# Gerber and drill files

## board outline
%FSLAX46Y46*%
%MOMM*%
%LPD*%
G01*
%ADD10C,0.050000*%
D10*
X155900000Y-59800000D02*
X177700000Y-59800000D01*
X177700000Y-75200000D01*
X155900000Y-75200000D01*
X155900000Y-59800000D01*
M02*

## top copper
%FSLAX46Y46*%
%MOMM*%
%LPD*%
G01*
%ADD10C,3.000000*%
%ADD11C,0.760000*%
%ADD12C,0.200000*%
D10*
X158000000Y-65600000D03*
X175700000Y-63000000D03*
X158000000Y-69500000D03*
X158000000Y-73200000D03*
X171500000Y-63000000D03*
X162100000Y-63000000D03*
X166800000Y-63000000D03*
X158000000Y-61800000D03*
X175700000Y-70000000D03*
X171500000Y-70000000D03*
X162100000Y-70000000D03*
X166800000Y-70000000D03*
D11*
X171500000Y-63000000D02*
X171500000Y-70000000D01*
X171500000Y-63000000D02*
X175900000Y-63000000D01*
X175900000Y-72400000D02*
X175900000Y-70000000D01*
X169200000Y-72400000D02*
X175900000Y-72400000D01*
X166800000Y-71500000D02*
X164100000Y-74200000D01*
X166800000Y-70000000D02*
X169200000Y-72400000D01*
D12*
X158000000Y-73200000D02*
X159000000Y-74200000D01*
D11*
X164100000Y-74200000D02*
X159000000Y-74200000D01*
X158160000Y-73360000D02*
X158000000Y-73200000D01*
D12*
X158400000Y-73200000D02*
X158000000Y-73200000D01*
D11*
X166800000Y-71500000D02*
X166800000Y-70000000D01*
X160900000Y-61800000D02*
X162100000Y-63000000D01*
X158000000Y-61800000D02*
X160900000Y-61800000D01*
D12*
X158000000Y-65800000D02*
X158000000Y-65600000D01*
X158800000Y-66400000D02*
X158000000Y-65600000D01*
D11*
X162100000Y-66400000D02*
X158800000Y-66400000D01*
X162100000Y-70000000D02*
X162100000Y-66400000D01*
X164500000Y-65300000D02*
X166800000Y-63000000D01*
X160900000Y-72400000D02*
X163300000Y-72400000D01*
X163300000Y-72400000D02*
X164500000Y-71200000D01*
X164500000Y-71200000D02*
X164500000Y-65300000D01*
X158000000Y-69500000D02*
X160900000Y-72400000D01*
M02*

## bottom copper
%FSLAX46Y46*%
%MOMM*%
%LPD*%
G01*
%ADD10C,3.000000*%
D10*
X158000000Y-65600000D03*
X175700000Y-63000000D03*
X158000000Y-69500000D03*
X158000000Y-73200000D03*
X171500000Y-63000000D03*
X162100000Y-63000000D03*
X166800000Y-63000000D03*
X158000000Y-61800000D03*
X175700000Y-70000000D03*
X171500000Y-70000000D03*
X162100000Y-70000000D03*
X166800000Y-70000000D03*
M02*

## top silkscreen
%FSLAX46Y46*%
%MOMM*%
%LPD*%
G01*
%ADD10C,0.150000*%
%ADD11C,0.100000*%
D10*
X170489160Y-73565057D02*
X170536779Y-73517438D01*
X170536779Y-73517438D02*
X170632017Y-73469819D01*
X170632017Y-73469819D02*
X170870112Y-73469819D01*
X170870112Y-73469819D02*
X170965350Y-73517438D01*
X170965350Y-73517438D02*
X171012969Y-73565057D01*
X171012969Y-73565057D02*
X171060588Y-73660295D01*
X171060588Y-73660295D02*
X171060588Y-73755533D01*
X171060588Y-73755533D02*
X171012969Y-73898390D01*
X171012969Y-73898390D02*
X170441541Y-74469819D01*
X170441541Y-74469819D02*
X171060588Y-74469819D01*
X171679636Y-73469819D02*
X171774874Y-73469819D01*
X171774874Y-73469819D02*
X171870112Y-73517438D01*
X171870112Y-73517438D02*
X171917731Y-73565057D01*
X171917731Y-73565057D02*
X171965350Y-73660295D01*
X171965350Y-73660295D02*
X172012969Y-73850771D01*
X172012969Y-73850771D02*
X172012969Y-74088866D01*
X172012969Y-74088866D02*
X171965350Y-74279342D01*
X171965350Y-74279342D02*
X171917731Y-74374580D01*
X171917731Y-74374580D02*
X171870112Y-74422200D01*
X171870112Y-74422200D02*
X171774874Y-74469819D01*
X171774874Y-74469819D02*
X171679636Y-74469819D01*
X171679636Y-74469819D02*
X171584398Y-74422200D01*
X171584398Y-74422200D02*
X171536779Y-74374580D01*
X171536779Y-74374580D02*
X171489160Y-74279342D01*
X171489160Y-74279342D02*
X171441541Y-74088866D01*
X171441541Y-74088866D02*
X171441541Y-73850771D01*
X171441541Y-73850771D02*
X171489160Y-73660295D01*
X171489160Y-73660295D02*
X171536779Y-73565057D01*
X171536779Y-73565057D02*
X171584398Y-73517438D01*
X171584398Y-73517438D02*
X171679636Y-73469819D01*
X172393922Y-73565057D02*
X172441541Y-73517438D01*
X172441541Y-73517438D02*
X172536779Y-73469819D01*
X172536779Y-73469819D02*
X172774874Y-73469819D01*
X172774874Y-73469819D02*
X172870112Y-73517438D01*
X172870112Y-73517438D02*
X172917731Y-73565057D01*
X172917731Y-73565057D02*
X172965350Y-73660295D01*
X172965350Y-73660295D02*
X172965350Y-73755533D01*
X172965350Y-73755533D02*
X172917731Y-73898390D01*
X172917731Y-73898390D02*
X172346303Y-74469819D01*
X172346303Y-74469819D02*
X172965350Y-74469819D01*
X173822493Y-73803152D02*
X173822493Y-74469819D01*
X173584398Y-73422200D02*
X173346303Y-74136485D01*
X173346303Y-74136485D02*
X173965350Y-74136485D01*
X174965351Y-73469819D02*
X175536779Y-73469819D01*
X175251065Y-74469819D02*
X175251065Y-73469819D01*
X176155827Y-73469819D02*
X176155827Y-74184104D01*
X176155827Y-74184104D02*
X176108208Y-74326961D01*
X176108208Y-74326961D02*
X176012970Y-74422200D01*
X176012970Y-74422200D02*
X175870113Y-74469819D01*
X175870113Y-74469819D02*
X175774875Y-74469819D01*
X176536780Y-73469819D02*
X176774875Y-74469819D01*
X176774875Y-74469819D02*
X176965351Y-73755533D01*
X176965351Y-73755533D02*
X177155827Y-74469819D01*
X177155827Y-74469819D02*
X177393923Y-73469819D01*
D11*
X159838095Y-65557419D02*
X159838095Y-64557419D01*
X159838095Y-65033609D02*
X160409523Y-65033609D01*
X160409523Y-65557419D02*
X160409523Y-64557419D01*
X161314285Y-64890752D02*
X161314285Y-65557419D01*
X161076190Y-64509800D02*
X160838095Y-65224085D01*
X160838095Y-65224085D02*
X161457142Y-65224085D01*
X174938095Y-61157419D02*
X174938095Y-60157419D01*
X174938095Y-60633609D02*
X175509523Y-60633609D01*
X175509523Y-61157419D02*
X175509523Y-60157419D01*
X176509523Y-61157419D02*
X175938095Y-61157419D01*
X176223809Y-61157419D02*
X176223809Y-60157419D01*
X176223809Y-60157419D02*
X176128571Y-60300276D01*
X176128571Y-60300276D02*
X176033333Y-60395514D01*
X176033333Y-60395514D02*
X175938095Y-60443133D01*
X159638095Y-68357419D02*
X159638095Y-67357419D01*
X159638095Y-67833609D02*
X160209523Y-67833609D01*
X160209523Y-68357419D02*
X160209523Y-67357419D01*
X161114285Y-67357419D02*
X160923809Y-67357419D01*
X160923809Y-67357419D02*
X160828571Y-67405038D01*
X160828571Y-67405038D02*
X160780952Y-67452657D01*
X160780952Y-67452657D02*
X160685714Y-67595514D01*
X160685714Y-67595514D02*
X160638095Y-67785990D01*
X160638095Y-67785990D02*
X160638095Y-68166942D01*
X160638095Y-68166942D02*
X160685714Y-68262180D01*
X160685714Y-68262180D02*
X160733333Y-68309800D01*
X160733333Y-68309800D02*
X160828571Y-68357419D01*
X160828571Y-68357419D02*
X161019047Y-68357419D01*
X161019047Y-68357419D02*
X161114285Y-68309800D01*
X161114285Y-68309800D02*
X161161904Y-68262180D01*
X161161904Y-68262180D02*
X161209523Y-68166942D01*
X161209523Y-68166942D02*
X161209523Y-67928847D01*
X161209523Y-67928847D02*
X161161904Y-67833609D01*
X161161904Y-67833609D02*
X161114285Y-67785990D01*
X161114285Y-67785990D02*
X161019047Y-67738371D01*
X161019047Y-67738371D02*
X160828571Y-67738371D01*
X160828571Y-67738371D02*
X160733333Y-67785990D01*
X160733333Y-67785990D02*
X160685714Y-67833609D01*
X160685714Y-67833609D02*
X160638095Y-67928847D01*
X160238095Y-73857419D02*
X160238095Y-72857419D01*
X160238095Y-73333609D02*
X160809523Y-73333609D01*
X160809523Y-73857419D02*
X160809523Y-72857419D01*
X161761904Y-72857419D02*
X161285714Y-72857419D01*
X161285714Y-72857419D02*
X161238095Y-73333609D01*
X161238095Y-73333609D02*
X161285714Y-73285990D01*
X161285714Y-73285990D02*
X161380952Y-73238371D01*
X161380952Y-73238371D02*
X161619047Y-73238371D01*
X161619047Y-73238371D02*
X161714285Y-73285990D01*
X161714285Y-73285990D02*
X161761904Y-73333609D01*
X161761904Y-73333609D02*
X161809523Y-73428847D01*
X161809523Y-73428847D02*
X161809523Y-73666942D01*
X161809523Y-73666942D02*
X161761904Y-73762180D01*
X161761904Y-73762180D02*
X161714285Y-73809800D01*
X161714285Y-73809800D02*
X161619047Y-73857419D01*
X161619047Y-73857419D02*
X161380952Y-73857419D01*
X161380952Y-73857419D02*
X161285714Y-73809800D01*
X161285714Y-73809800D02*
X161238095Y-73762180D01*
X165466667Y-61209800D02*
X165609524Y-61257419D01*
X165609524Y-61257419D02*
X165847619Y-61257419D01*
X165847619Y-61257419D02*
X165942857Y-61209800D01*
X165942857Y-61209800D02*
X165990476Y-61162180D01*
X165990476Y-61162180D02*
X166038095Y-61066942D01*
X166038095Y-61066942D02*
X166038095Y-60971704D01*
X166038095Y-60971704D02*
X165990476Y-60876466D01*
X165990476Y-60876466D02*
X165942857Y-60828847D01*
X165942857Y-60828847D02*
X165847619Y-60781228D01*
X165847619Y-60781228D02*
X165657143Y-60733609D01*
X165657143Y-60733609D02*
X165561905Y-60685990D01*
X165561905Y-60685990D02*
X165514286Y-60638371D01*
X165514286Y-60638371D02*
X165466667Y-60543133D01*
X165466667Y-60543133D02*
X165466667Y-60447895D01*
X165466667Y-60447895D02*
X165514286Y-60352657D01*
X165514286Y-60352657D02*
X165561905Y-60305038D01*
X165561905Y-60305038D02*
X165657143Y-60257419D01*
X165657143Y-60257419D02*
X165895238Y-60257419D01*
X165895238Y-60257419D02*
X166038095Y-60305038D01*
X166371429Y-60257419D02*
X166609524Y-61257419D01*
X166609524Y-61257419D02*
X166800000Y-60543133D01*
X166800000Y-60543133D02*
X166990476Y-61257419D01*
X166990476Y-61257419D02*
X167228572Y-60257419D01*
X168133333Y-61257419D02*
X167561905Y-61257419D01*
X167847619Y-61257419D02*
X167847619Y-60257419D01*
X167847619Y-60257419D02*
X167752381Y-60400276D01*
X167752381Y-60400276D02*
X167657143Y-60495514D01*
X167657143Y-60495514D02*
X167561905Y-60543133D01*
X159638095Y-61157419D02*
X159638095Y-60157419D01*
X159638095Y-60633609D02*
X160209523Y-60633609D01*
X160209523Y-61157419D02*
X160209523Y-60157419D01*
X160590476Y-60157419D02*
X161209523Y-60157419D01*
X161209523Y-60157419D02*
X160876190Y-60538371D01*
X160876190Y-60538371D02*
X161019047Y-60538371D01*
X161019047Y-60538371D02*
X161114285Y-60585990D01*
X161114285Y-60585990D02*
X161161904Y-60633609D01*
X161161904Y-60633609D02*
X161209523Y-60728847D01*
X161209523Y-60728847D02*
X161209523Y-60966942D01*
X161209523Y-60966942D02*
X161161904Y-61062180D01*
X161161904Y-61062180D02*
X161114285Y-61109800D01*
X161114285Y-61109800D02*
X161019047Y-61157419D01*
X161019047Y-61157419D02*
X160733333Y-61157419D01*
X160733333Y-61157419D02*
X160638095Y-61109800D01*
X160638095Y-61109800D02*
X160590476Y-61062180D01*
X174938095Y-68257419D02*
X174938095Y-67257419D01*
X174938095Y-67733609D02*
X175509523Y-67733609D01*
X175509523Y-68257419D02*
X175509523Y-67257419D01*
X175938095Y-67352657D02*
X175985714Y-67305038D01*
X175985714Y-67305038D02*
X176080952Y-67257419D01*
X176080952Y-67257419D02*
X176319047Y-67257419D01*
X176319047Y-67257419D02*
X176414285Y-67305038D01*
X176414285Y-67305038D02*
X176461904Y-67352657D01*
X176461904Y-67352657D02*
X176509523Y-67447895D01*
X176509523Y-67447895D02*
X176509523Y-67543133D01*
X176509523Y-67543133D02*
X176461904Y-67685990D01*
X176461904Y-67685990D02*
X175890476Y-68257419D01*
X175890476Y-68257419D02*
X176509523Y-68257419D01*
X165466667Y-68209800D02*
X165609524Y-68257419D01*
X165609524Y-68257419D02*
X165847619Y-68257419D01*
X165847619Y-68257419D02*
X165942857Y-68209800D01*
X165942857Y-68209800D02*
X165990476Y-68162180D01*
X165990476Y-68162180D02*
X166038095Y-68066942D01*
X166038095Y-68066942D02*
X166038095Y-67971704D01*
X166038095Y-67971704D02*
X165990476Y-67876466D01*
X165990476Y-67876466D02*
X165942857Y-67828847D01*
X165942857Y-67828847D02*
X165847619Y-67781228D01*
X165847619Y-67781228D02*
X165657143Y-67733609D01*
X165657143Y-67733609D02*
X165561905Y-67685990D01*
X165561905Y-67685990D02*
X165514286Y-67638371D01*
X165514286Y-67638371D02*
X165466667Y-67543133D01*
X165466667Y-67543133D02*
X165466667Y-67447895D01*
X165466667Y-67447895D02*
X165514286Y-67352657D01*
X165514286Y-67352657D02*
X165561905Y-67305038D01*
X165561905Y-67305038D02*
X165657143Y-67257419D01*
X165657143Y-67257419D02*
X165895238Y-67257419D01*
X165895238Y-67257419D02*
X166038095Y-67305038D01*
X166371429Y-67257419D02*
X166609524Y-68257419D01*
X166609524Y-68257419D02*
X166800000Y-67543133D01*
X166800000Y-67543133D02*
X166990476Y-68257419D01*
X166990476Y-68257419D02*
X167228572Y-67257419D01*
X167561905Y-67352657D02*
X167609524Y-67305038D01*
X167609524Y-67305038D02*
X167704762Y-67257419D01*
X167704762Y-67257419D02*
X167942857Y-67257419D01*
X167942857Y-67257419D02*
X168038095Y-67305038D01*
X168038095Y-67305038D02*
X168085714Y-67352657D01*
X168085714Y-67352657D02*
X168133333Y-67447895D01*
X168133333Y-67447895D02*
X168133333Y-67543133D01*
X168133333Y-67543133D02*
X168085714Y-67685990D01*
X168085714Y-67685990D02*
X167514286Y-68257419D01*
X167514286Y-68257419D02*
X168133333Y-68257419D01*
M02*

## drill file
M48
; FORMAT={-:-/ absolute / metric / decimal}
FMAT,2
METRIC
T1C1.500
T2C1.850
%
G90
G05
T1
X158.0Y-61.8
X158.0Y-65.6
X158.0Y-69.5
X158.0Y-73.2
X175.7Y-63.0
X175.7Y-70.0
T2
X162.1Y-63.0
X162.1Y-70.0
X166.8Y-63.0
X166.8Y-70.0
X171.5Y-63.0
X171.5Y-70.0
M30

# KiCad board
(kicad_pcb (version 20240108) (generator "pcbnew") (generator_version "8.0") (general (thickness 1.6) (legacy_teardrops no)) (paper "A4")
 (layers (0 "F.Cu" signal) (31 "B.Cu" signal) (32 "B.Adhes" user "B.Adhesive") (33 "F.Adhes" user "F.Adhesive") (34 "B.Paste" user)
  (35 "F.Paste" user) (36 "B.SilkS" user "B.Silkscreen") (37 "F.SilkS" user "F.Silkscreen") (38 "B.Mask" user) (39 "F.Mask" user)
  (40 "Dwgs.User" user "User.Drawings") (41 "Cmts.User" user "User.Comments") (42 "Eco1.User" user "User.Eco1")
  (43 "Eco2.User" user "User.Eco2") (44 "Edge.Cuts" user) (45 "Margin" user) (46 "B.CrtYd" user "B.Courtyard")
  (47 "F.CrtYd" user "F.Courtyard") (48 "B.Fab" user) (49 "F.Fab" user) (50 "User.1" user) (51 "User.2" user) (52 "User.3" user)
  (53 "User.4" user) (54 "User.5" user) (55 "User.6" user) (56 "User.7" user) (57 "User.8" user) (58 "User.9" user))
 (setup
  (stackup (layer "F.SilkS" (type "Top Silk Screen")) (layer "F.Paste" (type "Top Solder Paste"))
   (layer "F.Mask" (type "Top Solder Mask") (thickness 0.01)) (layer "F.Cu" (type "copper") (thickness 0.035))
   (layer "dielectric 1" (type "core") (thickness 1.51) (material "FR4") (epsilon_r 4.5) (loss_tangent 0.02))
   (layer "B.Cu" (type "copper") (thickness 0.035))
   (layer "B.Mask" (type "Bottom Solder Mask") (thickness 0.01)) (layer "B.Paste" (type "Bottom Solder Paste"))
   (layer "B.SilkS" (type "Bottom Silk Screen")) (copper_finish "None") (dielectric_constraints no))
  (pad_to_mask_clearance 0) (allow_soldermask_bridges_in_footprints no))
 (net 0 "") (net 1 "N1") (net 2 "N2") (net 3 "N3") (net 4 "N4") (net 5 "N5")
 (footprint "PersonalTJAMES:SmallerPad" (layer "F.Cu") (at 158 65.5)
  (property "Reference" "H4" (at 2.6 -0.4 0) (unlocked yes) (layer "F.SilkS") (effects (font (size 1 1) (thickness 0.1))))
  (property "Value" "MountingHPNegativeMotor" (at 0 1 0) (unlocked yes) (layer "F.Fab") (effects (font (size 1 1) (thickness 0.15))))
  (pad "1" thru_hole circle (at 0 0.1) (size 3 3) (drill 1.5) (layers "*.Cu" "*.Mask") (remove_unused_layers no) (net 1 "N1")))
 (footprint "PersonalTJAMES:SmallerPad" (layer "F.Cu") (at 175.7 62.9)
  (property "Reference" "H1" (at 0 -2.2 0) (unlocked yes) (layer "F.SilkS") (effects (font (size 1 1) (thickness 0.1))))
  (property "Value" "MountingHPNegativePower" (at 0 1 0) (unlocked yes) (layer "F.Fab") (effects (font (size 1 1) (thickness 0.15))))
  (pad "1" thru_hole circle (at 0 0.1) (size 3 3) (drill 1.5) (layers "*.Cu" "*.Mask") (remove_unused_layers no) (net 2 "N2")))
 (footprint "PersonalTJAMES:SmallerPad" (layer "F.Cu") (at 158 69.4)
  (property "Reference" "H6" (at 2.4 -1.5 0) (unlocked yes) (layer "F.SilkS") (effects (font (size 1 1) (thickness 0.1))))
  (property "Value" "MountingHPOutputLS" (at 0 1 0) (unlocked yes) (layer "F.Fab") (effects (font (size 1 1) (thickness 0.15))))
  (pad "1" thru_hole circle (at 0 0.1) (size 3 3) (drill 1.5) (layers "*.Cu" "*.Mask") (remove_unused_layers no) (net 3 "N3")))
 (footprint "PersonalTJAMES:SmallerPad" (layer "F.Cu") (at 158 73.1)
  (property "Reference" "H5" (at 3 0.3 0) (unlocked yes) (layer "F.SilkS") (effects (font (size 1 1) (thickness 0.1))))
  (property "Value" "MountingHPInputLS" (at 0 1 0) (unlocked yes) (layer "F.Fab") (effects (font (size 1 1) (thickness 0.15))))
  (pad "1" thru_hole circle (at 0 0.1) (size 3 3) (drill 1.5) (layers "*.Cu" "*.Mask") (remove_unused_layers no) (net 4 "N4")))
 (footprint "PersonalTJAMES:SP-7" (layer "F.Cu") (at 166.8 63)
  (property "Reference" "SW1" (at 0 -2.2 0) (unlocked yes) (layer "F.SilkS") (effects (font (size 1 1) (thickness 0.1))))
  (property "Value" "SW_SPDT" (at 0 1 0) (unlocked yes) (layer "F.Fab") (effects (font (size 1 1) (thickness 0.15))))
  (pad "1" thru_hole circle (at 4.7 0) (size 3 3) (drill 1.85) (layers "*.Cu" "*.Mask") (remove_unused_layers no) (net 2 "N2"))
  (pad "2" thru_hole circle (at -4.7 0) (size 3 3) (drill 1.85) (layers "*.Cu" "*.Mask") (remove_unused_layers no) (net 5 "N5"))
  (pad "3" thru_hole circle (at 0 0) (size 3 3) (drill 1.85) (layers "*.Cu" "*.Mask") (remove_unused_layers no) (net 3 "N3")))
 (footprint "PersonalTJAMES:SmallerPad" (layer "F.Cu") (at 158 61.7)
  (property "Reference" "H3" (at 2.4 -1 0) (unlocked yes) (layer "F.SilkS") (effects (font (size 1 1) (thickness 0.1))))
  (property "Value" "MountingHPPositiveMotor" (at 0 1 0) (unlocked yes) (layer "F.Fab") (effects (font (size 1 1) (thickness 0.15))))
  (pad "1" thru_hole circle (at 0 0.1) (size 3 3) (drill 1.5) (layers "*.Cu" "*.Mask") (remove_unused_layers no) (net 5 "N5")))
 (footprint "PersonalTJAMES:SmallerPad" (layer "F.Cu") (at 175.7 69.9)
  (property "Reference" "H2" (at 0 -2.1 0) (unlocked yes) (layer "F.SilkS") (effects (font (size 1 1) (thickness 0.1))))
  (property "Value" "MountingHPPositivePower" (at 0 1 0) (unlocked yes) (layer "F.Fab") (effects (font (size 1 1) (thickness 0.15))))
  (pad "1" thru_hole circle (at 0 0.1) (size 3 3) (drill 1.5) (layers "*.Cu" "*.Mask") (remove_unused_layers no) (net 4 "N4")))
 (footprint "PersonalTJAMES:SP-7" (layer "F.Cu") (at 166.8 70)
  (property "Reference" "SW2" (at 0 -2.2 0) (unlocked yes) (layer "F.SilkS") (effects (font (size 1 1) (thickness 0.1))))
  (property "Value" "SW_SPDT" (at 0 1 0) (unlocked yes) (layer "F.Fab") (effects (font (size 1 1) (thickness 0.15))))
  (pad "1" thru_hole circle (at 4.7 0) (size 3 3) (drill 1.85) (layers "*.Cu" "*.Mask") (remove_unused_layers no) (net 2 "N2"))
  (pad "2" thru_hole circle (at -4.7 0) (size 3 3) (drill 1.85) (layers "*.Cu" "*.Mask") (remove_unused_layers no) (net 1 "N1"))
  (pad "3" thru_hole circle (at 0 0) (size 3 3) (drill 1.85) (layers "*.Cu" "*.Mask") (remove_unused_layers no) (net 4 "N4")))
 (gr_rect (start 155.9 59.8) (end 177.7 75.2) (stroke (width 0.05) (type default)) (fill none) (layer "Edge.Cuts"))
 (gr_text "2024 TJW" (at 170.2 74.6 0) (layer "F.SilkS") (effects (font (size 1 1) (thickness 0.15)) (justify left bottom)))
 (segment (start 171.5 63) (end 171.5 70) (width 0.76) (layer "F.Cu") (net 2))
 (segment (start 171.5 63) (end 175.9 63) (width 0.76) (layer "F.Cu") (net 2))
 (segment (start 175.9 72.4) (end 175.9 70) (width 0.76) (layer "F.Cu") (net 4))
 (segment (start 169.2 72.4) (end 175.9 72.4) (width 0.76) (layer "F.Cu") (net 4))
 (segment (start 166.8 71.5) (end 164.1 74.2) (width 0.76) (layer "F.Cu") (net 4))
 (segment (start 166.8 70) (end 169.2 72.4) (width 0.76) (layer "F.Cu") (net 4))
 (segment (start 158 73.2) (end 159 74.2) (width 0.2) (layer "F.Cu") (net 4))
 (segment (start 164.1 74.2) (end 159 74.2) (width 0.76) (layer "F.Cu") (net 4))
 (segment (start 158.16 73.36) (end 158 73.2) (width 0.76) (layer "F.Cu") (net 4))
 (segment (start 158.4 73.2) (end 158 73.2) (width 0.2) (layer "F.Cu") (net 4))
 (segment (start 166.8 71.5) (end 166.8 70) (width 0.76) (layer "F.Cu") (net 4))
 (segment (start 160.9 61.8) (end 162.1 63) (width 0.76) (layer "F.Cu") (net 5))
 (segment (start 158 61.8) (end 160.9 61.8) (width 0.76) (layer "F.Cu") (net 5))
 (segment (start 158 65.8) (end 158 65.6) (width 0.2) (layer "F.Cu") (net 1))
 (segment (start 158.8 66.4) (end 158 65.6) (width 0.2) (layer "F.Cu") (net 1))
 (segment (start 162.1 66.4) (end 158.8 66.4) (width 0.76) (layer "F.Cu") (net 1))
 (segment (start 162.1 70) (end 162.1 66.4) (width 0.76) (layer "F.Cu") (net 1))
 (segment (start 164.5 65.3) (end 166.8 63) (width 0.76) (layer "F.Cu") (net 3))
 (segment (start 160.9 72.4) (end 163.3 72.4) (width 0.76) (layer "F.Cu") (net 3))
 (segment (start 163.3 72.4) (end 164.5 71.2) (width 0.76) (layer "F.Cu") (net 3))
 (segment (start 164.5 71.2) (end 164.5 65.3) (width 0.76) (layer "F.Cu") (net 3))
 (segment (start 158 69.5) (end 160.9 72.4) (width 0.76) (layer "F.Cu") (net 3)))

